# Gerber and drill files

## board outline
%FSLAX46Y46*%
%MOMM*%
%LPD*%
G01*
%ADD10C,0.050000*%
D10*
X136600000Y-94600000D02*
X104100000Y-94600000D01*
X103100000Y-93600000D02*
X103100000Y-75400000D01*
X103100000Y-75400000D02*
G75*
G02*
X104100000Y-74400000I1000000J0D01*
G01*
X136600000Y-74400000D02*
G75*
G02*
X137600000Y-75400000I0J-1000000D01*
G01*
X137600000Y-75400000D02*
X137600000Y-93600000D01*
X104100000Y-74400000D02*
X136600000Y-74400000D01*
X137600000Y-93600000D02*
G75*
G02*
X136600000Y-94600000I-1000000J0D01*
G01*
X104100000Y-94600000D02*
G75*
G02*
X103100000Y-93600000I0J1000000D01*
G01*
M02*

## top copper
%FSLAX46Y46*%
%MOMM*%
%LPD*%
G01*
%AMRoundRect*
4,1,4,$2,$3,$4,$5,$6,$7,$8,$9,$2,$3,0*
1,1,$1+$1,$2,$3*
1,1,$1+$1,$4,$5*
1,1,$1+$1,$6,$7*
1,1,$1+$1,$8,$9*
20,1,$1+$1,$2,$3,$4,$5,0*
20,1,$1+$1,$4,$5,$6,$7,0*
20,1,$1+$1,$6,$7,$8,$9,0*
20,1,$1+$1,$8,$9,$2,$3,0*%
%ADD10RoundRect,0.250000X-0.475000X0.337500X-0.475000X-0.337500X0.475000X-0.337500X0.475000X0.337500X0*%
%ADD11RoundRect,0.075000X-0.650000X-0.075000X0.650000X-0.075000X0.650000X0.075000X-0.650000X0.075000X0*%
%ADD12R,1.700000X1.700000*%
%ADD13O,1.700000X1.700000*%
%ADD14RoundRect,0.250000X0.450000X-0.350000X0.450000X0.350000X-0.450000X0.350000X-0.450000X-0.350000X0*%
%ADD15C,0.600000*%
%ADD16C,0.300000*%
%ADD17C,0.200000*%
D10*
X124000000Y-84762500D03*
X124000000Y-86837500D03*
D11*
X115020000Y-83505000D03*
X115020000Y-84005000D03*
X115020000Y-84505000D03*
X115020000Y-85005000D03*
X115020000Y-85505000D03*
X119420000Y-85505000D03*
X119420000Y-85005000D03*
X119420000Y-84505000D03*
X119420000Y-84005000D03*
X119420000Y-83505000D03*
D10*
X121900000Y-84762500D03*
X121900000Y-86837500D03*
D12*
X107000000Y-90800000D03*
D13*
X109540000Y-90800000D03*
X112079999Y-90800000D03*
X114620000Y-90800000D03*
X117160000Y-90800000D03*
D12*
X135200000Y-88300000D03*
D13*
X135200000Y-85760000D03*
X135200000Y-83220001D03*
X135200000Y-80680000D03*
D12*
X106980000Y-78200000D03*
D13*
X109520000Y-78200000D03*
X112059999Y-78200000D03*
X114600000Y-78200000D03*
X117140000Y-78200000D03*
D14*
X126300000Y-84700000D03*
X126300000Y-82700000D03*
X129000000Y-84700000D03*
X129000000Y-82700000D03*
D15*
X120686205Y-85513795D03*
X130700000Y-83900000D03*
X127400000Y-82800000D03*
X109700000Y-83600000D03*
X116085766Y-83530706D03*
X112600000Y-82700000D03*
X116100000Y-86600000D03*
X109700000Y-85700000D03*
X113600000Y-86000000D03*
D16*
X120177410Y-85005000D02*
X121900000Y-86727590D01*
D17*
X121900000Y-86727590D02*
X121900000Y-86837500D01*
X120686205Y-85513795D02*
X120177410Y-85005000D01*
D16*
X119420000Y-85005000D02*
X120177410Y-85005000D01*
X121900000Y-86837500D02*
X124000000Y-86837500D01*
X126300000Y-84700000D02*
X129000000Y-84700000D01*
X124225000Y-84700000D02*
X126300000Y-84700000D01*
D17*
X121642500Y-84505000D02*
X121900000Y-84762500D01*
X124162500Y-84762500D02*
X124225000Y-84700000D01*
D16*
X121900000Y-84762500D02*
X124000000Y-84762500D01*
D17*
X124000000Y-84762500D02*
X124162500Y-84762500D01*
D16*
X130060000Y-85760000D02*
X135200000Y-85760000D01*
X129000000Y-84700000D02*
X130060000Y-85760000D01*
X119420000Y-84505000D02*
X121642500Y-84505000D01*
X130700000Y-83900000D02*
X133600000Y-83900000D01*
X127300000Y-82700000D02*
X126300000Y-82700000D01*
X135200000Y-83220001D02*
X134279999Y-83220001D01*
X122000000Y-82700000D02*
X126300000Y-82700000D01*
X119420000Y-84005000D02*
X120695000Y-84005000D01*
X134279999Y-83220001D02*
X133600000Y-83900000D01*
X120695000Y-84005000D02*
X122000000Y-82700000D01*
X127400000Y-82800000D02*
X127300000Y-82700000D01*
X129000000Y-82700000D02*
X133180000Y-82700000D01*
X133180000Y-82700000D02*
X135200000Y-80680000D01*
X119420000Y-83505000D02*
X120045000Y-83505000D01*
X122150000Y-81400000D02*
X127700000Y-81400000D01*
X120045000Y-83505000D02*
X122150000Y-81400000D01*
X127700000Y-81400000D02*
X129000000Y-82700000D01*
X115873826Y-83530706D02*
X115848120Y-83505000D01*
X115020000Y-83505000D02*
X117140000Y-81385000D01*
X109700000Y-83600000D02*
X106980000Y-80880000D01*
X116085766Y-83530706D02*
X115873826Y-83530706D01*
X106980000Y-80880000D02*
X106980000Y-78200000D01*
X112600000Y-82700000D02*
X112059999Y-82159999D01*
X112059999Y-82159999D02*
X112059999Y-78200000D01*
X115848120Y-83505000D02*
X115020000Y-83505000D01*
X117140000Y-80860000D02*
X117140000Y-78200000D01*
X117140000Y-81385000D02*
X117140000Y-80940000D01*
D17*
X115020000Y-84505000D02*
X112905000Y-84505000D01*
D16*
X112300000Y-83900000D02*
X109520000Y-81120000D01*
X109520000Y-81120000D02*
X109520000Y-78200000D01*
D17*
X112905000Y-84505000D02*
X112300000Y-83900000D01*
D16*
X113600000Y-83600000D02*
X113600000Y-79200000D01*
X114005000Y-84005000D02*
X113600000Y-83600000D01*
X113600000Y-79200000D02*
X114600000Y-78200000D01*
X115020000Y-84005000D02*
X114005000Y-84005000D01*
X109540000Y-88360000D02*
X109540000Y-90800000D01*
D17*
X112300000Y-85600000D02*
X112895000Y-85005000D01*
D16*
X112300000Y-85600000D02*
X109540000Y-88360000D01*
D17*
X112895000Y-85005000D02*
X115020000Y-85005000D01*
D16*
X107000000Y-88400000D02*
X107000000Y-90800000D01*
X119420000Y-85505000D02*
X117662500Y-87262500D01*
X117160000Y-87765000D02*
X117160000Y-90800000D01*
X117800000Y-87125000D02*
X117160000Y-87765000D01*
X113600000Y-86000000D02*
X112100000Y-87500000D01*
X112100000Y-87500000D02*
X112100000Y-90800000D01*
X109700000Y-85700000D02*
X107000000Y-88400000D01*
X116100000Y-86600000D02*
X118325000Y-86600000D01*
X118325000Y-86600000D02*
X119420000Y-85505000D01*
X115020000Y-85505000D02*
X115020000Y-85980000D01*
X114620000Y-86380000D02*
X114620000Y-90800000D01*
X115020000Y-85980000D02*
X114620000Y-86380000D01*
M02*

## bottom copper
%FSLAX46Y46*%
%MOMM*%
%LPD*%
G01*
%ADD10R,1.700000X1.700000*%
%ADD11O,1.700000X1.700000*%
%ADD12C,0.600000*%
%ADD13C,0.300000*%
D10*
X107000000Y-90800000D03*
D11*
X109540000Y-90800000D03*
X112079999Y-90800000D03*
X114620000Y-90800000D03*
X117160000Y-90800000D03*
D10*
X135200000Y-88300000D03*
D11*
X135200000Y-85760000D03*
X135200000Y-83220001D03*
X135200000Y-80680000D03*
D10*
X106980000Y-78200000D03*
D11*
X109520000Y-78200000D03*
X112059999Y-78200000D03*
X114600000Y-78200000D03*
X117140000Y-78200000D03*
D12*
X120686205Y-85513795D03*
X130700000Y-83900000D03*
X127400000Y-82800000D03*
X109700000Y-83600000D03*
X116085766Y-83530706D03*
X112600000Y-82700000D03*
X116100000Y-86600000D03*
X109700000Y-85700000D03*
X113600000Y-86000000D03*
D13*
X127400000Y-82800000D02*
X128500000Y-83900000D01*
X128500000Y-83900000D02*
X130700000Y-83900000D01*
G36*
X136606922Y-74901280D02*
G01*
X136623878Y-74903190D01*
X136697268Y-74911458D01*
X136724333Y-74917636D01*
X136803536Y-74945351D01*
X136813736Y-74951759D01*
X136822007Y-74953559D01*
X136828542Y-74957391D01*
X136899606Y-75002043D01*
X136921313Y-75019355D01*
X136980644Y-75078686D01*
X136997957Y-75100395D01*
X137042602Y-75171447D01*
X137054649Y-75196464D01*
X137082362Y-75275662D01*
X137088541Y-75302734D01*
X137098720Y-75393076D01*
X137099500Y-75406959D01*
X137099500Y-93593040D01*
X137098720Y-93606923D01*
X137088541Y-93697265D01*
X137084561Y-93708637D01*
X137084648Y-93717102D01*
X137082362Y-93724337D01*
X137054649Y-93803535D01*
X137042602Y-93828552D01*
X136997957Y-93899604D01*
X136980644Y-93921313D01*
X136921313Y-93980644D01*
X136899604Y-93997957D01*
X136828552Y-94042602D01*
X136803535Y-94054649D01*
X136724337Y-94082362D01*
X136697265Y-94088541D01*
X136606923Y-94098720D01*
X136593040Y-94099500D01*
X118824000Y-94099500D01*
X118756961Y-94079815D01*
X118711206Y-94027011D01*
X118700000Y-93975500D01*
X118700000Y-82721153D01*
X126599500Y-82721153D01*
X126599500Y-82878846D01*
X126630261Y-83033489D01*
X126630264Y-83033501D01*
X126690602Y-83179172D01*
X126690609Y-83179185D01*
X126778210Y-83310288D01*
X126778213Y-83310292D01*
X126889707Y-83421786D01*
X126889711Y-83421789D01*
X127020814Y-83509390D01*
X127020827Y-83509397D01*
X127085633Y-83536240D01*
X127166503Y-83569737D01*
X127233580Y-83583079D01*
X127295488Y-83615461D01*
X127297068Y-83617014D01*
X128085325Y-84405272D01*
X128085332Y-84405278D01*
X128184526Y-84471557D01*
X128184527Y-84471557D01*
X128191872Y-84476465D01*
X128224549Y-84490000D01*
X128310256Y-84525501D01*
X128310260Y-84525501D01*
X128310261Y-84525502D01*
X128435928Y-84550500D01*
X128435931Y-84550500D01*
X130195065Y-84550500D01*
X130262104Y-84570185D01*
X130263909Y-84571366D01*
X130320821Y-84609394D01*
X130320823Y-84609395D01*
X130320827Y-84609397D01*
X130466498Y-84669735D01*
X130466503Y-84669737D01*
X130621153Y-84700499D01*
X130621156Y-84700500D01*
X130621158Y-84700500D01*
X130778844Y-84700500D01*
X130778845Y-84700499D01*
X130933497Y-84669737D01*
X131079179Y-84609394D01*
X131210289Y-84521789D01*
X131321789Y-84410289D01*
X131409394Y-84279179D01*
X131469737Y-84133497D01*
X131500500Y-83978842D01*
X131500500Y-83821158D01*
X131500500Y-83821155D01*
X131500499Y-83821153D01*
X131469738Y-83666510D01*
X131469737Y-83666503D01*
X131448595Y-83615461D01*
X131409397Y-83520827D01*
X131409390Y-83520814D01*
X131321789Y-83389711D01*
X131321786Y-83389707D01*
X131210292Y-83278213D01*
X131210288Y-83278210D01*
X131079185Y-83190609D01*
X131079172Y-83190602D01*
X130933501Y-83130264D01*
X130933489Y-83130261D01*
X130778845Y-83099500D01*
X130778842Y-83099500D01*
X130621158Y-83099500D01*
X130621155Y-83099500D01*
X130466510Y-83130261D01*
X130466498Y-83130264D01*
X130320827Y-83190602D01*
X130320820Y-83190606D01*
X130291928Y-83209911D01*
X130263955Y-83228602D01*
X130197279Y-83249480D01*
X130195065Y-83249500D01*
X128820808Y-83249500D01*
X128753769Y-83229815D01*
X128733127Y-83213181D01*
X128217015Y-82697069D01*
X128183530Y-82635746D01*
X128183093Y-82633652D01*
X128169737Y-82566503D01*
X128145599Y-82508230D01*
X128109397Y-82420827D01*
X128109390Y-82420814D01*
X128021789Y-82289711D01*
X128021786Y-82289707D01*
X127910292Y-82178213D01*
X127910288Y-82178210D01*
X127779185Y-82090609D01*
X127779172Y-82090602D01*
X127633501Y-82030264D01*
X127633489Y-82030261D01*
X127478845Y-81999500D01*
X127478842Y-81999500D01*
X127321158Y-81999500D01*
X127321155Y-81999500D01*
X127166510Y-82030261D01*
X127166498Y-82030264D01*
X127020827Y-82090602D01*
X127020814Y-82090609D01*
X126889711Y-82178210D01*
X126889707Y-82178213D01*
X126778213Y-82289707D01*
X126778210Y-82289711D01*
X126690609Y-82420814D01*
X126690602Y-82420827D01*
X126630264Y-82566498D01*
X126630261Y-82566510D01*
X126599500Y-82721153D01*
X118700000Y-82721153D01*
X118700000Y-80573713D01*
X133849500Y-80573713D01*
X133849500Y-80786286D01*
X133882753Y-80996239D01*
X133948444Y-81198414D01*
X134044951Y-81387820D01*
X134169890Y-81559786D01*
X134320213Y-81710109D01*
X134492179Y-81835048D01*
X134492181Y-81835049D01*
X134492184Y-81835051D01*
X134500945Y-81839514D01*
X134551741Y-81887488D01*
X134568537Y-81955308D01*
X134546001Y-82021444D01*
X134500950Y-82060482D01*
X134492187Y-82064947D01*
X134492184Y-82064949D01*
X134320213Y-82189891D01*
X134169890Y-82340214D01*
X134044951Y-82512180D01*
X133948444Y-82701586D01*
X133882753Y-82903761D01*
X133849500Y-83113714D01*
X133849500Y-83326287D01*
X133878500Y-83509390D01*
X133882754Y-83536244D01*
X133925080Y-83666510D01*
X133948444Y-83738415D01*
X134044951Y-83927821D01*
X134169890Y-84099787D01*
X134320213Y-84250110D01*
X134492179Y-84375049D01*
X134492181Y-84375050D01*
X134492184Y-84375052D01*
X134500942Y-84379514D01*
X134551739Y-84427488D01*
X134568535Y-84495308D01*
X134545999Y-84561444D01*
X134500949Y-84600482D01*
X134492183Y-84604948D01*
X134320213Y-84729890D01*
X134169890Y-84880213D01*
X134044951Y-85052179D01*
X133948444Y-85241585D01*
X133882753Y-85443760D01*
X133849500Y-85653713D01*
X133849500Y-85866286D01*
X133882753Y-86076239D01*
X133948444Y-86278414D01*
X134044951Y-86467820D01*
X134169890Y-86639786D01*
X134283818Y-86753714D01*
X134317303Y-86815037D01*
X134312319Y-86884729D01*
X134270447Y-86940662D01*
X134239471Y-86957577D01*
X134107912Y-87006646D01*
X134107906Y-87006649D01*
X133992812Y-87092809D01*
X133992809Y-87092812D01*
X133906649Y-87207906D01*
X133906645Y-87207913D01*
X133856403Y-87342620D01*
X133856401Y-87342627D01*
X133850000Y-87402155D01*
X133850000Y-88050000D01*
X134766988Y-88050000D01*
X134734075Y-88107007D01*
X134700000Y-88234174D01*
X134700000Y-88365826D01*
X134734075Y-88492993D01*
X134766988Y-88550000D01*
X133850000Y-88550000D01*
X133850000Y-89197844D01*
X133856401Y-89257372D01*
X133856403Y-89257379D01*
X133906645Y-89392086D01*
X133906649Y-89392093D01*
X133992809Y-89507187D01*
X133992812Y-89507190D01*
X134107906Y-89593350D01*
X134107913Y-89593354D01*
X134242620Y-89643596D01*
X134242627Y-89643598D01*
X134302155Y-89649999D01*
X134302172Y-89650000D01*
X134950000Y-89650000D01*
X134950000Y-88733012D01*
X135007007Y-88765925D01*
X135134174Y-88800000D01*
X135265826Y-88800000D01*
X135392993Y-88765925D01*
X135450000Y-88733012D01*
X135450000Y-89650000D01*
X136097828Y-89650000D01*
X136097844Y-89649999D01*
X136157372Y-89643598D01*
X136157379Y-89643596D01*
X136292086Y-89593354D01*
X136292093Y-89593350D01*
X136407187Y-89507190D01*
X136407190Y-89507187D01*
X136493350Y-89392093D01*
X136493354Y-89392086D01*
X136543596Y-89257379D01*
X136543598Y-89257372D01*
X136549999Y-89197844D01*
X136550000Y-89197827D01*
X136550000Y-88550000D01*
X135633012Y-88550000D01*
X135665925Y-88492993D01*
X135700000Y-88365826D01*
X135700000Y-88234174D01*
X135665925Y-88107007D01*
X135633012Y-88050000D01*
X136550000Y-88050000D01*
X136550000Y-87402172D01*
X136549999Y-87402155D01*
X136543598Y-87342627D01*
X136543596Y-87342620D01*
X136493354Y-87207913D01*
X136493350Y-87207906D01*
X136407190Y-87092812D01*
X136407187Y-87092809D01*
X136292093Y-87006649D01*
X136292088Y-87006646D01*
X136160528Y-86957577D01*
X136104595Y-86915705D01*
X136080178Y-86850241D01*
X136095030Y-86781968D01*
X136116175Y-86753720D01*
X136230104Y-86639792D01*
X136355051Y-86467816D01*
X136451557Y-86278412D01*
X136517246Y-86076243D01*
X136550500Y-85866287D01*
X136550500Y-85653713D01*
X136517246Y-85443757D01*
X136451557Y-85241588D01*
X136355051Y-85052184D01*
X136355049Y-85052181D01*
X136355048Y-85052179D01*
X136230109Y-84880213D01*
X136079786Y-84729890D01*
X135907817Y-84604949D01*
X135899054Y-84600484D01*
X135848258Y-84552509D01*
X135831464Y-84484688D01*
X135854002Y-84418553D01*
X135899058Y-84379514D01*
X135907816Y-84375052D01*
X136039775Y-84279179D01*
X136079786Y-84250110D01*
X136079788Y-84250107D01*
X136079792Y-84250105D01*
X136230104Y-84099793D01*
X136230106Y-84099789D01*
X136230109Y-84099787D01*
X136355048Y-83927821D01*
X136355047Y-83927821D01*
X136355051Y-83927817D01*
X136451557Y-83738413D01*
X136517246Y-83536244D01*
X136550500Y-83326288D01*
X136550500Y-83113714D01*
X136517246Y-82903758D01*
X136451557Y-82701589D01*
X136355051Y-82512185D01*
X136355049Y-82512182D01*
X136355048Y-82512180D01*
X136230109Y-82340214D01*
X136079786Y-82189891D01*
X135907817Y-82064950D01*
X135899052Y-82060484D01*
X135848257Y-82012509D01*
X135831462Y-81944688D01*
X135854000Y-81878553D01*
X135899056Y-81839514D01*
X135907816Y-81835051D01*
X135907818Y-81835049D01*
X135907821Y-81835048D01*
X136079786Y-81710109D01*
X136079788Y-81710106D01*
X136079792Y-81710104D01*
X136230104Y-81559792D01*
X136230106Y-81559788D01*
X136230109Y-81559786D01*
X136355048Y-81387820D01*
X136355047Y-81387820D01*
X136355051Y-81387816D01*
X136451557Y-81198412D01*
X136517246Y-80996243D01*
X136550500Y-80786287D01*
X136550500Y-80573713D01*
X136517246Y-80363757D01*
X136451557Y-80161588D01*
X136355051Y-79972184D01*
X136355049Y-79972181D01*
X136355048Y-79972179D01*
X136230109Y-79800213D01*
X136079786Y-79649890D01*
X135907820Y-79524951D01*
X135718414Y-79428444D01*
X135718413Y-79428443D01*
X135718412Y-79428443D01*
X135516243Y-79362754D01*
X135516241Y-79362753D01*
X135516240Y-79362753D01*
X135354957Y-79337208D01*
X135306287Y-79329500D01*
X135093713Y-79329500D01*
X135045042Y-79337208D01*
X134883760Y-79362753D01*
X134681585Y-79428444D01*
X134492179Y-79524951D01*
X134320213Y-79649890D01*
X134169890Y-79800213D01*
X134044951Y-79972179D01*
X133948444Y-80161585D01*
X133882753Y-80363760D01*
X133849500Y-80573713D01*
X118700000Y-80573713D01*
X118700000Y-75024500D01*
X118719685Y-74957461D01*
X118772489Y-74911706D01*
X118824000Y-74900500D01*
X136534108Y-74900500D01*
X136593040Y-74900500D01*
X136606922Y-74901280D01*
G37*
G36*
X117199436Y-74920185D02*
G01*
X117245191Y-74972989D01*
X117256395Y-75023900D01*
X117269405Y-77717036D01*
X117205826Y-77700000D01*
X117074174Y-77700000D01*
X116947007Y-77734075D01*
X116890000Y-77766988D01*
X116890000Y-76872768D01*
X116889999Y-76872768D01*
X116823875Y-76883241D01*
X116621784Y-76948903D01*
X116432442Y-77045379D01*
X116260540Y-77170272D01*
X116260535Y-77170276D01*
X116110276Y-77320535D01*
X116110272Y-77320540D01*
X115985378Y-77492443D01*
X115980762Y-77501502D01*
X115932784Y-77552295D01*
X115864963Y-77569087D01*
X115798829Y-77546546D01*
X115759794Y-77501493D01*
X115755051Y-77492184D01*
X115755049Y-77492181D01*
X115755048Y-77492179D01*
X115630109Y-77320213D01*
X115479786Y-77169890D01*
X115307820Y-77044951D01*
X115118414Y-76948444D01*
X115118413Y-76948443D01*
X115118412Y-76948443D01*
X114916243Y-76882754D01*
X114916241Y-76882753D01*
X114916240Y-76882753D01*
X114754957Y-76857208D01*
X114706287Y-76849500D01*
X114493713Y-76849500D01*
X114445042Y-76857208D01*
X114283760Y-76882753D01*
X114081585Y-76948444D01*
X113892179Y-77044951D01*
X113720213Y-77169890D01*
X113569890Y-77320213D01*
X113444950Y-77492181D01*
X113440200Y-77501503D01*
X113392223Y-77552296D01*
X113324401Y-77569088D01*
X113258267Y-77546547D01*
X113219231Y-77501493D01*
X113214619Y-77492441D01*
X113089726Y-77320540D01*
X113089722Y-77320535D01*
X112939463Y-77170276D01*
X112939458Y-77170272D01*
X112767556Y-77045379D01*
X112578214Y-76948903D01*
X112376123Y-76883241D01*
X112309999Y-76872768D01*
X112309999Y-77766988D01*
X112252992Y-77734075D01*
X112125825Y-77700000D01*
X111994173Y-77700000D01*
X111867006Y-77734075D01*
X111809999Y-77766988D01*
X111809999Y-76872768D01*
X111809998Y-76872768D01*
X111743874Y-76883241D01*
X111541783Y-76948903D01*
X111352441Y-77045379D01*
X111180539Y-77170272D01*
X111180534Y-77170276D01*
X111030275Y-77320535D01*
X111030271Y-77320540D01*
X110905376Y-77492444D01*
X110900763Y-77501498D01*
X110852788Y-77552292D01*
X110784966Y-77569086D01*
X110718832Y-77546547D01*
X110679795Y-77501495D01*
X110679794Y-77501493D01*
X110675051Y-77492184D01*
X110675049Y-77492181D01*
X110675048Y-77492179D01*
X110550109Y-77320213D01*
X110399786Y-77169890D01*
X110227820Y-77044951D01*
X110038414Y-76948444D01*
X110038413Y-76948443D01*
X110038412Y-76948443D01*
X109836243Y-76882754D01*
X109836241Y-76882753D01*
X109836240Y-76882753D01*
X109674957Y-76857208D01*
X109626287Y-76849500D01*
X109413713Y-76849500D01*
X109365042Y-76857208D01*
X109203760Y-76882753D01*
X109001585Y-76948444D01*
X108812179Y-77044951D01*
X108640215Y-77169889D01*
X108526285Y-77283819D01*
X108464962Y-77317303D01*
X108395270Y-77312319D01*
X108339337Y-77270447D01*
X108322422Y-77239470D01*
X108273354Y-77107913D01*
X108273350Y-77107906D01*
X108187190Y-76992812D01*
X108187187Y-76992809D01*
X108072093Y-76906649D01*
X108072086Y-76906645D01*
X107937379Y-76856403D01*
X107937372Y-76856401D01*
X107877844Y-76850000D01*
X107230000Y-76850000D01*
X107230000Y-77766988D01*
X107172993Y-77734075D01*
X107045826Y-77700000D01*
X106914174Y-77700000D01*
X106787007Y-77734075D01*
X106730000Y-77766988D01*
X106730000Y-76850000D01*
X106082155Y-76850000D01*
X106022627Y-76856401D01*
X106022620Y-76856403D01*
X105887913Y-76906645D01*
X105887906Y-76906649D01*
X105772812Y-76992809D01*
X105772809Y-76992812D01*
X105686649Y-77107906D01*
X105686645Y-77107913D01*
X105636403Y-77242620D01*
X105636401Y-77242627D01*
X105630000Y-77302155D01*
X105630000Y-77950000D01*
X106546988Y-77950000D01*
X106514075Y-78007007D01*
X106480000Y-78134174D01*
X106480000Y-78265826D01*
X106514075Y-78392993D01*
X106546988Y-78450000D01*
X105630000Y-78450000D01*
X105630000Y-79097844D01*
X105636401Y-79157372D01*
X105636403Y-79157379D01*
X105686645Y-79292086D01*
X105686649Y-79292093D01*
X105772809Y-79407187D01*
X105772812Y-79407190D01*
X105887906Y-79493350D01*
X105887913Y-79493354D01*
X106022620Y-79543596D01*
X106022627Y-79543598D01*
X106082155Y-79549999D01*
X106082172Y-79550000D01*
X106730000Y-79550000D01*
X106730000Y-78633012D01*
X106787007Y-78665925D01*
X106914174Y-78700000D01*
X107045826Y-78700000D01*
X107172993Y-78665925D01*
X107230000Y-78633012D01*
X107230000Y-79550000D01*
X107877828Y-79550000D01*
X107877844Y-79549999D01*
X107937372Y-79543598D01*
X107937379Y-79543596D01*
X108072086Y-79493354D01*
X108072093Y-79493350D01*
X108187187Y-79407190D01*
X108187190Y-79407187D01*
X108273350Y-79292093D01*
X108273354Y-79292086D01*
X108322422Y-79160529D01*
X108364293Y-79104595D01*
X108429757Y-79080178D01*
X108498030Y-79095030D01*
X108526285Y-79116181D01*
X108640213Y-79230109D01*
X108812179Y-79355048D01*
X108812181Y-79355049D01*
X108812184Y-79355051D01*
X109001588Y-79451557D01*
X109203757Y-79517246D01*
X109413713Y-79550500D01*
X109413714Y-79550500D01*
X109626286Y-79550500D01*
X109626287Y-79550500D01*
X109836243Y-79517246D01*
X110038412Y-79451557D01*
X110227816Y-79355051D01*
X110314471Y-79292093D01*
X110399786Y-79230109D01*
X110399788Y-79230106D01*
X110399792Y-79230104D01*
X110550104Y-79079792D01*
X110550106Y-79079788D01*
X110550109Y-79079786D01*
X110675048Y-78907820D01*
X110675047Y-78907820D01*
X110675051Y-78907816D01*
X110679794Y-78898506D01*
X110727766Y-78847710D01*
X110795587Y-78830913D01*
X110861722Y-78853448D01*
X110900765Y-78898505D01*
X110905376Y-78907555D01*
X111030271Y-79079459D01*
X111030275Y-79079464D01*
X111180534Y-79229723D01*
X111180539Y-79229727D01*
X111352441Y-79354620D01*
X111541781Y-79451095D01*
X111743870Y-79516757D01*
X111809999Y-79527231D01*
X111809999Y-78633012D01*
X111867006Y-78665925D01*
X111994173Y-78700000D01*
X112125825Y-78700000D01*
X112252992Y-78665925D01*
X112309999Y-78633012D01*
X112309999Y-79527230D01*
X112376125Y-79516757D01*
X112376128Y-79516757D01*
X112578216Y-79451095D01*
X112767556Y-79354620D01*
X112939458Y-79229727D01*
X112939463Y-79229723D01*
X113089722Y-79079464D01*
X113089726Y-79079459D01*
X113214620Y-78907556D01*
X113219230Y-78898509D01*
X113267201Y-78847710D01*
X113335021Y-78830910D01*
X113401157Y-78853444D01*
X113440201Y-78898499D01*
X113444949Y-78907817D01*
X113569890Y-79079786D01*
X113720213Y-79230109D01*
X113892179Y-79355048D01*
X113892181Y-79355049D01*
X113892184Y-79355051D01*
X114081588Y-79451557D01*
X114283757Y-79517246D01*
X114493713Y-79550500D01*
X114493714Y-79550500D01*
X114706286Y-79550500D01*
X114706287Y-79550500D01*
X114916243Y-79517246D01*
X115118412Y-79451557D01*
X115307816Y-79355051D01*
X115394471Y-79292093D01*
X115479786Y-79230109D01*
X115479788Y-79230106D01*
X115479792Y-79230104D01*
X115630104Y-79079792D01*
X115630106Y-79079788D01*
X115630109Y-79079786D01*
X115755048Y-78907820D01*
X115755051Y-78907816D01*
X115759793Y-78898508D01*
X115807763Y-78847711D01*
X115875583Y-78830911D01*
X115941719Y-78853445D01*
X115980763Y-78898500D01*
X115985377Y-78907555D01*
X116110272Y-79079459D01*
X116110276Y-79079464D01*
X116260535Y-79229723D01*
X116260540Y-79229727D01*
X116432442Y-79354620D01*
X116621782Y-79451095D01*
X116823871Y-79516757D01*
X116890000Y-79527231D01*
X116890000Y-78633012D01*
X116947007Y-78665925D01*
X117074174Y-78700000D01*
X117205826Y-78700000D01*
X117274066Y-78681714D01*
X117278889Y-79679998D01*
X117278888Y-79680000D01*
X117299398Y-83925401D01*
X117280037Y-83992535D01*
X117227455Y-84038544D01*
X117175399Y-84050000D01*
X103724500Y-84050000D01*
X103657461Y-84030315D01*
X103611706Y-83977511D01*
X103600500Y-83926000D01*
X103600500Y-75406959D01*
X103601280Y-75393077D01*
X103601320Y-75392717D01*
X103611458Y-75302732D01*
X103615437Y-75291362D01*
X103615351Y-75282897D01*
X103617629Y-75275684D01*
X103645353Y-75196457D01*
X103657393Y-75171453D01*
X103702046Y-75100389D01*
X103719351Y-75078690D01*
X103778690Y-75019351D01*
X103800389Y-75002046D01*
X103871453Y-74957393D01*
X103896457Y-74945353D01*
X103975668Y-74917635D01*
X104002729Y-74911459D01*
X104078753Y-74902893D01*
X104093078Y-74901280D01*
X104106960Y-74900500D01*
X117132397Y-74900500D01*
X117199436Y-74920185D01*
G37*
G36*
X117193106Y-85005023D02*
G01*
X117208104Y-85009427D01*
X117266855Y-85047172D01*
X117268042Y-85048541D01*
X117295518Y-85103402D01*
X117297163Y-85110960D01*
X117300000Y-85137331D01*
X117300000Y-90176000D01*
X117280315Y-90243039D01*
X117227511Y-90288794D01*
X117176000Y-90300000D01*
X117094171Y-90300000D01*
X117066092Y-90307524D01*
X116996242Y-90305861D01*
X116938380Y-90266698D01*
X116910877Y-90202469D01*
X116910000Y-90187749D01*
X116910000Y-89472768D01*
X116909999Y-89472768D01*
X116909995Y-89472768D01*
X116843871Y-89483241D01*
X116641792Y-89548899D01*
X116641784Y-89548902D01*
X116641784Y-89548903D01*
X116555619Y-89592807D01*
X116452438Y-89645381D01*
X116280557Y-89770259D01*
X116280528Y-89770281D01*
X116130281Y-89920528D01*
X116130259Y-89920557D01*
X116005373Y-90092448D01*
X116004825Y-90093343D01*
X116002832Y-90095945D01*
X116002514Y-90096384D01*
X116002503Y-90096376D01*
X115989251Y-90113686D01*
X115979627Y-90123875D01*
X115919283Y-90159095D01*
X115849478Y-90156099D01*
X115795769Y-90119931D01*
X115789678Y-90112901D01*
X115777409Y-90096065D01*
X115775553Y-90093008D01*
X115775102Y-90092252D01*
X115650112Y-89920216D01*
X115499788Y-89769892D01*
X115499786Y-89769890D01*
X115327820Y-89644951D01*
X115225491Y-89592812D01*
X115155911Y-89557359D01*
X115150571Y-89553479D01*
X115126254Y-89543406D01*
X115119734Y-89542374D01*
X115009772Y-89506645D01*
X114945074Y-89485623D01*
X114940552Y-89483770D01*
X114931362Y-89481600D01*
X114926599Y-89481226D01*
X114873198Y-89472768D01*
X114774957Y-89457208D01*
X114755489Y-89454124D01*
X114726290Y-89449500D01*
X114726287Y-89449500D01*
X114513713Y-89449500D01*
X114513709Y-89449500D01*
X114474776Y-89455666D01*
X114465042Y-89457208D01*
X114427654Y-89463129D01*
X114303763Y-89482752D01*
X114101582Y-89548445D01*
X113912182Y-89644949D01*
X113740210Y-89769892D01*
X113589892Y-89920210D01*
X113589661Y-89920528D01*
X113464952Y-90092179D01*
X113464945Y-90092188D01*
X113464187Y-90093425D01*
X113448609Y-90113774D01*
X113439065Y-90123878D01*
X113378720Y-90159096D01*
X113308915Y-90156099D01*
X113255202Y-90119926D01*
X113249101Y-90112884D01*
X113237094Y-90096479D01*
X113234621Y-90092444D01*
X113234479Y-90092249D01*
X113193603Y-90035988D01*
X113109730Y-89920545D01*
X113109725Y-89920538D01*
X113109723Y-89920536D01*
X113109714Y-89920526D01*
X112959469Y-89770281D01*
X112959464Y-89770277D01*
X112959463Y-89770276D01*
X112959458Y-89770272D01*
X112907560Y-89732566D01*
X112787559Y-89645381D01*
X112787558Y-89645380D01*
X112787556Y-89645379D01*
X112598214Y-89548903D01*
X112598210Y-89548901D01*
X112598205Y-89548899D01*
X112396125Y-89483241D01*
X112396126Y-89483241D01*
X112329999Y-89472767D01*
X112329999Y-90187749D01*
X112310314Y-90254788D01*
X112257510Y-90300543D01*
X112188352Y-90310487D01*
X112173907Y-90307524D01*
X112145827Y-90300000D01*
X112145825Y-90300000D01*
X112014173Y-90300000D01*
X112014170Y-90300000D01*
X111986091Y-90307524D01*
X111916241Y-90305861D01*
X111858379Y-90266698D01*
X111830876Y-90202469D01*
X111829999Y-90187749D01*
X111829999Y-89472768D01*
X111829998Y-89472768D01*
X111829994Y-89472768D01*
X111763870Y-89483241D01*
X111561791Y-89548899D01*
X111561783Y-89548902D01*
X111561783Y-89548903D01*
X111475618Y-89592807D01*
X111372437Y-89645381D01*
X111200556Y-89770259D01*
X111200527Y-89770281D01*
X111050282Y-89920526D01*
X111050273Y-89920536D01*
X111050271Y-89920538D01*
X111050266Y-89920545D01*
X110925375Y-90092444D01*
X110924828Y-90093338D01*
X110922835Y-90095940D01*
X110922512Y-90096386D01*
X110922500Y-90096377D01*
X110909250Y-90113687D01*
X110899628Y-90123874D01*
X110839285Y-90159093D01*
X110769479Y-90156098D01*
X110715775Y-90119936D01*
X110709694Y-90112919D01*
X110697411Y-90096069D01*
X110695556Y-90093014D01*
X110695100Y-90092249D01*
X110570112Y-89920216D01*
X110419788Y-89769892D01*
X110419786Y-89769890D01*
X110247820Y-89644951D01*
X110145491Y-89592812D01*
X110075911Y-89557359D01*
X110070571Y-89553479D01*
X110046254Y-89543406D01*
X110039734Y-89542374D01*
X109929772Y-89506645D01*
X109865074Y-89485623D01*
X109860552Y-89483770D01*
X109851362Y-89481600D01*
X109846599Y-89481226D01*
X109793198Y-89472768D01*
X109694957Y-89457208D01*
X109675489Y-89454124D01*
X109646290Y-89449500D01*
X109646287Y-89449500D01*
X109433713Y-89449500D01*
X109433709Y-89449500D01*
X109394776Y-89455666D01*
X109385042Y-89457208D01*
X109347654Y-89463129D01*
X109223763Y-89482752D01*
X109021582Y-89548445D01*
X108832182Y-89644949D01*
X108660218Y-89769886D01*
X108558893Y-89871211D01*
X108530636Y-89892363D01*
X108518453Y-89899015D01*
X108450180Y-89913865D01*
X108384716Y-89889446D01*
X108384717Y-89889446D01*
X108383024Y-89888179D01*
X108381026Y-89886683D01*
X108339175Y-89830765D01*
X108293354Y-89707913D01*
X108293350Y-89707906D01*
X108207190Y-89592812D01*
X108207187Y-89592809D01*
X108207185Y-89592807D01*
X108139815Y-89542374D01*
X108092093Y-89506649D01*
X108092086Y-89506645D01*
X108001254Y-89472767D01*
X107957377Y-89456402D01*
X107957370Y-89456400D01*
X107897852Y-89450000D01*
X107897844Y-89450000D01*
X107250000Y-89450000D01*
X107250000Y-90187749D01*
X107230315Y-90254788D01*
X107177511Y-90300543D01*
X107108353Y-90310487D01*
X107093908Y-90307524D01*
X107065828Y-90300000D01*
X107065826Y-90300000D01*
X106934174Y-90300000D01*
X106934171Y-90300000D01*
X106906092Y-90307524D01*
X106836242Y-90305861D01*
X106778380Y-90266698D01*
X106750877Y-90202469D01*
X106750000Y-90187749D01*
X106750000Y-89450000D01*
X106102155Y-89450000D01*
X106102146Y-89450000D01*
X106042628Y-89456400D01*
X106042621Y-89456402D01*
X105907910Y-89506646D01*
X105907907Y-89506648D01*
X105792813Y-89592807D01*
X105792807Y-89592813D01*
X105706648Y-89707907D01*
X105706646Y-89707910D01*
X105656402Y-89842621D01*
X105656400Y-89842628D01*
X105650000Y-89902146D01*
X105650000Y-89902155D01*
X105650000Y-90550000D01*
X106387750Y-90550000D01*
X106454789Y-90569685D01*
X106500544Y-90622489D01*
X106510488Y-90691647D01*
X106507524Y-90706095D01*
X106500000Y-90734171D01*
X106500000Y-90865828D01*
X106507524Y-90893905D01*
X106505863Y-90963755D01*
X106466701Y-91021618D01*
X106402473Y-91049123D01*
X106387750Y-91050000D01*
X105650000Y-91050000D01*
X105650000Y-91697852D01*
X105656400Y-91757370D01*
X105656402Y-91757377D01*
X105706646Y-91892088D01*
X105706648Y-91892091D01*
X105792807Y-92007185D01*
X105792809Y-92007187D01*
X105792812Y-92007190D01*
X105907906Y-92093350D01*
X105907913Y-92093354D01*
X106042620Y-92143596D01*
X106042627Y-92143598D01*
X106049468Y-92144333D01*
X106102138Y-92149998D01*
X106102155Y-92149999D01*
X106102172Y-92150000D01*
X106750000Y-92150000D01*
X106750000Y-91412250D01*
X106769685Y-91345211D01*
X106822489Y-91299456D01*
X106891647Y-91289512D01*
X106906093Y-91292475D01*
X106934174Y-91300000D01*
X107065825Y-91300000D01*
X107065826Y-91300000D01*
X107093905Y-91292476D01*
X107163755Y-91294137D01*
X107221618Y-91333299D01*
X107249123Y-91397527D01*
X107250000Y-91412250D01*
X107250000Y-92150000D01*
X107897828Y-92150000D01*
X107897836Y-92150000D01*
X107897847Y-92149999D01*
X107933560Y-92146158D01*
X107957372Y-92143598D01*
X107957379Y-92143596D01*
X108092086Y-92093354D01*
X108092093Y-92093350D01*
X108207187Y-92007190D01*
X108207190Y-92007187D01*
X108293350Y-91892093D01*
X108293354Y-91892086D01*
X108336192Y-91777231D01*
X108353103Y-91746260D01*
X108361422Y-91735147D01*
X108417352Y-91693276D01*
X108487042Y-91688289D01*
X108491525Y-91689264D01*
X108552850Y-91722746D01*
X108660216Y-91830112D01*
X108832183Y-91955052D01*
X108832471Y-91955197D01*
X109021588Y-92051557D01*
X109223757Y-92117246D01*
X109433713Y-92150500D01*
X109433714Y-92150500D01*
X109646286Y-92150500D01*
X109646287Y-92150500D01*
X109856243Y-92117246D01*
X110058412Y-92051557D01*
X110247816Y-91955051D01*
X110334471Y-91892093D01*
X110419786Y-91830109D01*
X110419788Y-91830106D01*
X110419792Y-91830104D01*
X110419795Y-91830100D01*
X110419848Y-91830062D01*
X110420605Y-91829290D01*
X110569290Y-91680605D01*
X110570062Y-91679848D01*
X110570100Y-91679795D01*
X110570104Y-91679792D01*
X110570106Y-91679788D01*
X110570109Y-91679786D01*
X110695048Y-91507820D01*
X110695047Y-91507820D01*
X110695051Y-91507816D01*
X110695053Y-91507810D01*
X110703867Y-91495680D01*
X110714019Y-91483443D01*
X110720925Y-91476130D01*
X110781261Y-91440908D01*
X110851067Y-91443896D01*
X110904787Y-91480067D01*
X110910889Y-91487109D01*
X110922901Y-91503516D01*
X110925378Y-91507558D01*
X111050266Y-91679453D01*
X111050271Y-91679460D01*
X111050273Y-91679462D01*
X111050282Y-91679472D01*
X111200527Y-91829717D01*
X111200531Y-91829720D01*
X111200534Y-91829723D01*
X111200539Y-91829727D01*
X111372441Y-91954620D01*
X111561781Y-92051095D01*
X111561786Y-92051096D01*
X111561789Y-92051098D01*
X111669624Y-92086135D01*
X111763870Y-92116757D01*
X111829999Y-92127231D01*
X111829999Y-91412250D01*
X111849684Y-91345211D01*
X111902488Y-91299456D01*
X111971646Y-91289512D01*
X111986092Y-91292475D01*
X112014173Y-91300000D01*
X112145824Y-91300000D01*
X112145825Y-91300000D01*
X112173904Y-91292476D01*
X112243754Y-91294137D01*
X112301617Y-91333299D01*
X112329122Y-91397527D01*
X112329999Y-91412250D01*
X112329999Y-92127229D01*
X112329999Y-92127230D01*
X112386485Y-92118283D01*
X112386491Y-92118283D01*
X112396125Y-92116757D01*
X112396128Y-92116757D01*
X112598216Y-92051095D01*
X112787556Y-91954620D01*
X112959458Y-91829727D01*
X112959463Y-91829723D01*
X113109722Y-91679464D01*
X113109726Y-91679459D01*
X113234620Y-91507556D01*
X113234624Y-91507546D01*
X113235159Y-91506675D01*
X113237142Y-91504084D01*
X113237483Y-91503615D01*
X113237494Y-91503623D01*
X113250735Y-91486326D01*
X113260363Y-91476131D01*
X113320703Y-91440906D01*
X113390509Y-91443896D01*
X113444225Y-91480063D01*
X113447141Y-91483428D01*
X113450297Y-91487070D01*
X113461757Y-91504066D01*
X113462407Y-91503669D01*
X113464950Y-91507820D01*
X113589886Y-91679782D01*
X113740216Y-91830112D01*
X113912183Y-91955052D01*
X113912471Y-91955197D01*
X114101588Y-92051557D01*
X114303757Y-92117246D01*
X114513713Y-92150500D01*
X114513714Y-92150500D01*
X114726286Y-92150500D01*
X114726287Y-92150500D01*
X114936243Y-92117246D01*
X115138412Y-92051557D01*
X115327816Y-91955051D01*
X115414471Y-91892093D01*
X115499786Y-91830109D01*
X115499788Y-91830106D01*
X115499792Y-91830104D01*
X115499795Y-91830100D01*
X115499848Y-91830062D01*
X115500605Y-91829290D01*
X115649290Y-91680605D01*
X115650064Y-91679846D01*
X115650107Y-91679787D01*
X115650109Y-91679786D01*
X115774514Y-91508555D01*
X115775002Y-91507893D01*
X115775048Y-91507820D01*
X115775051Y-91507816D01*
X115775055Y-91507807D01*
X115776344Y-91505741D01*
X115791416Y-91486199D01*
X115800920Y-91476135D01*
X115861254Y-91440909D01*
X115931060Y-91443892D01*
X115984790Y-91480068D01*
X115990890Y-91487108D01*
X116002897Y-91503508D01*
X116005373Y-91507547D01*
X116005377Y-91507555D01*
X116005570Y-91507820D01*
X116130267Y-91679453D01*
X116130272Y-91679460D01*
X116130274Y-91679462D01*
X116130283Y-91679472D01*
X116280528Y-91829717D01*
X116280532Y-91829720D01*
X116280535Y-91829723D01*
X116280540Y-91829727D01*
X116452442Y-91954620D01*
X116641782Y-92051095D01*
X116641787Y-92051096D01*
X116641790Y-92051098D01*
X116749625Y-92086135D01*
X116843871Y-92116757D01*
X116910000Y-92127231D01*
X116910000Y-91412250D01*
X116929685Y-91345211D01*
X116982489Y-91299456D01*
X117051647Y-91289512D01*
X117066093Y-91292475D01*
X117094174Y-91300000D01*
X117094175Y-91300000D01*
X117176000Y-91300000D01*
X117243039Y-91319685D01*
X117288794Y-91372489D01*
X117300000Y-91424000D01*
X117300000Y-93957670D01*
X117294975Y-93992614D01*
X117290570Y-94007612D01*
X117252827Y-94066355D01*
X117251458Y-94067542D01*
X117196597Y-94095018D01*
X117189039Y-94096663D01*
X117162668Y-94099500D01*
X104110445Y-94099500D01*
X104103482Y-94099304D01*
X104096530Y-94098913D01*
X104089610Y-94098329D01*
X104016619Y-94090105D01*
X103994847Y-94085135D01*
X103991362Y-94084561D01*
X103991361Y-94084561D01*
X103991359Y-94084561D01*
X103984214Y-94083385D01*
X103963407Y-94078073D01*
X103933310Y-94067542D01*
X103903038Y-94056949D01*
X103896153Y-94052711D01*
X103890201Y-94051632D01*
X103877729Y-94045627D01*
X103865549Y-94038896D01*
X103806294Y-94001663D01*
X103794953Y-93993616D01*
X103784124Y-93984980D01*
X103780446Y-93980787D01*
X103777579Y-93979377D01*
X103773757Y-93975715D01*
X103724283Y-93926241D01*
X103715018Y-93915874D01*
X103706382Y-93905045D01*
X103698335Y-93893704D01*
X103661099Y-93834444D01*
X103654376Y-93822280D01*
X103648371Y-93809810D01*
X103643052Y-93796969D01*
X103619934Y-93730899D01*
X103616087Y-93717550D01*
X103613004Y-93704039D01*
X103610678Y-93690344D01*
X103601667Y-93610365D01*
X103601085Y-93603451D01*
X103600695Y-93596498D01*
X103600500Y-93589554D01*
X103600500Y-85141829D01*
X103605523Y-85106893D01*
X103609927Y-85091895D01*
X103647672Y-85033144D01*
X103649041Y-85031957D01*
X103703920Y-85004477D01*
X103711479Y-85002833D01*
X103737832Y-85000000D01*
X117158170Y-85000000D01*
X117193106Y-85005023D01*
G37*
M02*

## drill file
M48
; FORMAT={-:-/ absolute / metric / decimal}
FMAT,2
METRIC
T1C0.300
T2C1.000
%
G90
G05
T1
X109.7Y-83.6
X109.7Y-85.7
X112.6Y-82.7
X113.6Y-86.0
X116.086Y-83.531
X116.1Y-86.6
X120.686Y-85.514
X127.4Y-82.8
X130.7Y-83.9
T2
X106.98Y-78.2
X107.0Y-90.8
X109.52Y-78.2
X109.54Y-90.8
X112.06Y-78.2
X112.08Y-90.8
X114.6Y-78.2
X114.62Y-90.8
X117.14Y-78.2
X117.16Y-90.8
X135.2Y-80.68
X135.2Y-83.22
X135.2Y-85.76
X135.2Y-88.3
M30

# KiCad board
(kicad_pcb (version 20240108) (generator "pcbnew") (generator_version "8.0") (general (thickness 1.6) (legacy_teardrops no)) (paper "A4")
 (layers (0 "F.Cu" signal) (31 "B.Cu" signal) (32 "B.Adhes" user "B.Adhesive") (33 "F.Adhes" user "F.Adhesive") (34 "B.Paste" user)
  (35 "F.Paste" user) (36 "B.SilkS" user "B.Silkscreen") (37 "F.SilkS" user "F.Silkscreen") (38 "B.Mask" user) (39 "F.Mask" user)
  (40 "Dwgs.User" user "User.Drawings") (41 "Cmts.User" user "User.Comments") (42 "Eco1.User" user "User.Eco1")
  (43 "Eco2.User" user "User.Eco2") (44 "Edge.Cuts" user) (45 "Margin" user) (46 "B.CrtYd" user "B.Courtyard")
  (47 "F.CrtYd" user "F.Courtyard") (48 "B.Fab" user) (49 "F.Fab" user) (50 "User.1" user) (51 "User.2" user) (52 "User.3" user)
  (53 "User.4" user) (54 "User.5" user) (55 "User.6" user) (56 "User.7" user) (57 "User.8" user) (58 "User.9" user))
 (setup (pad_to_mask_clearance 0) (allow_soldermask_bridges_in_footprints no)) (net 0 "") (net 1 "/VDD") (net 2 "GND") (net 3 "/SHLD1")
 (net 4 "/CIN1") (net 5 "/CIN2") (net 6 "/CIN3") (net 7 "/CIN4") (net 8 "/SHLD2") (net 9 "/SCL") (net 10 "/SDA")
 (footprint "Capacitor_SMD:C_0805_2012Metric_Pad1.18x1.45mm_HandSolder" (layer "F.Cu") (at 124 85.8 -90)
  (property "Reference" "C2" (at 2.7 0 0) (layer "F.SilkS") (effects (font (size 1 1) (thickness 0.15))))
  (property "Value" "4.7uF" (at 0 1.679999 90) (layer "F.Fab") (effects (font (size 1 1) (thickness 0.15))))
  (pad "1" smd roundrect (at -1.0375 0 270) (size 1.175 1.45) (layers "F.Cu" "F.Paste" "F.Mask") (roundrect_rratio 0.212766) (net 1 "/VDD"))
  (pad "2" smd roundrect (at 1.0375 0 270) (size 1.175 1.45) (layers "F.Cu" "F.Paste" "F.Mask") (roundrect_rratio 0.212766) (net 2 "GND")))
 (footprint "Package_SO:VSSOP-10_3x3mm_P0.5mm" (layer "F.Cu") (at 117.22 84.505)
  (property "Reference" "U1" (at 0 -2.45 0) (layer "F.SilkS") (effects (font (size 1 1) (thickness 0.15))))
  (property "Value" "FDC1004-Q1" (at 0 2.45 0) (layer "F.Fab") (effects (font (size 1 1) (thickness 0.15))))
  (pad "1" smd roundrect (at -2.2 -1) (size 1.45 0.3) (layers "F.Cu" "F.Paste" "F.Mask") (roundrect_rratio 0.25) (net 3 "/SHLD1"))
  (pad "2" smd roundrect (at -2.2 -0.5) (size 1.45 0.3) (layers "F.Cu" "F.Paste" "F.Mask") (roundrect_rratio 0.25) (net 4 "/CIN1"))
  (pad "3" smd roundrect (at -2.2 0) (size 1.45 0.3) (layers "F.Cu" "F.Paste" "F.Mask") (roundrect_rratio 0.25) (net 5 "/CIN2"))
  (pad "4" smd roundrect (at -2.2 0.5) (size 1.45 0.3) (layers "F.Cu" "F.Paste" "F.Mask") (roundrect_rratio 0.25) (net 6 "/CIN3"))
  (pad "5" smd roundrect (at -2.2 1) (size 1.45 0.3) (layers "F.Cu" "F.Paste" "F.Mask") (roundrect_rratio 0.25) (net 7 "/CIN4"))
  (pad "6" smd roundrect (at 2.2 1) (size 1.45 0.3) (layers "F.Cu" "F.Paste" "F.Mask") (roundrect_rratio 0.25) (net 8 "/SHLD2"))
  (pad "7" smd roundrect (at 2.2 0.5) (size 1.45 0.3) (layers "F.Cu" "F.Paste" "F.Mask") (roundrect_rratio 0.25) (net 2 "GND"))
  (pad "8" smd roundrect (at 2.2 0) (size 1.45 0.3) (layers "F.Cu" "F.Paste" "F.Mask") (roundrect_rratio 0.25) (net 1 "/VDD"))
  (pad "9" smd roundrect (at 2.2 -0.5) (size 1.45 0.3) (layers "F.Cu" "F.Paste" "F.Mask") (roundrect_rratio 0.25) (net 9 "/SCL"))
  (pad "10" smd roundrect (at 2.2 -1) (size 1.45 0.3) (layers "F.Cu" "F.Paste" "F.Mask") (roundrect_rratio 0.25) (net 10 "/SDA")))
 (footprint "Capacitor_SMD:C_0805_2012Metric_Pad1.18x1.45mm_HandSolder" (layer "F.Cu") (at 121.9 85.8 -90)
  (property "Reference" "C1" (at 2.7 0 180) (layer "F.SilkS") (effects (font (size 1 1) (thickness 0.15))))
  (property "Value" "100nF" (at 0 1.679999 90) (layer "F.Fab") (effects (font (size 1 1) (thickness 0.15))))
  (pad "1" smd roundrect (at -1.0375 0 270) (size 1.175 1.45) (layers "F.Cu" "F.Paste" "F.Mask") (roundrect_rratio 0.212766) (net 1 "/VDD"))
  (pad "2" smd roundrect (at 1.0375 0 270) (size 1.175 1.45) (layers "F.Cu" "F.Paste" "F.Mask") (roundrect_rratio 0.212766) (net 2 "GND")))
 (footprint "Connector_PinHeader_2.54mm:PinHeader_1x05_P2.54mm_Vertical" (layer "F.Cu") (at 107 90.8 90)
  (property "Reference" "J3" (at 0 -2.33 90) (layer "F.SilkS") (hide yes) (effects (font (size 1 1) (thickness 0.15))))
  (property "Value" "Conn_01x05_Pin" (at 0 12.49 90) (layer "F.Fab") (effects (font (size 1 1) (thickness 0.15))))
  (pad "1" thru_hole rect (at 0 0 90) (size 1.7 1.7) (drill 1) (layers "*.Cu" "*.Mask") (remove_unused_layers no) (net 8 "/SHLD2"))
  (pad "2" thru_hole oval (at 0 2.54 90) (size 1.7 1.7) (drill 1) (layers "*.Cu" "*.Mask") (remove_unused_layers no) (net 6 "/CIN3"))
  (pad "3" thru_hole oval (at 0 5.079999 90) (size 1.7 1.7) (drill 1) (layers "*.Cu" "*.Mask") (remove_unused_layers no) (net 8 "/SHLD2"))
  (pad "4" thru_hole oval (at 0 7.62 90) (size 1.7 1.7) (drill 1) (layers "*.Cu" "*.Mask") (remove_unused_layers no) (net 7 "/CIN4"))
  (pad "5" thru_hole oval (at 0 10.16 90) (size 1.7 1.7) (drill 1) (layers "*.Cu" "*.Mask") (remove_unused_layers no) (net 8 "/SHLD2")))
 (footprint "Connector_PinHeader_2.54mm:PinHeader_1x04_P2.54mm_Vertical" (layer "F.Cu") (at 135.2 88.3 180)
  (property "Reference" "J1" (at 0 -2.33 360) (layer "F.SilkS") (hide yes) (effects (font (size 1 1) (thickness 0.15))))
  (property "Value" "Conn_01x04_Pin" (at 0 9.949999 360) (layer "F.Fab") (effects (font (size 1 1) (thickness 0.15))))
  (pad "1" thru_hole rect (at 0 0 180) (size 1.7 1.7) (drill 1) (layers "*.Cu" "*.Mask") (remove_unused_layers no) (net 2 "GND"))
  (pad "2" thru_hole oval (at 0 2.54 180) (size 1.7 1.7) (drill 1) (layers "*.Cu" "*.Mask") (remove_unused_layers no) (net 1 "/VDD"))
  (pad "3" thru_hole oval (at 0 5.079999 180) (size 1.7 1.7) (drill 1) (layers "*.Cu" "*.Mask") (remove_unused_layers no) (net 9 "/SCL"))
  (pad "4" thru_hole oval (at 0 7.62 180) (size 1.7 1.7) (drill 1) (layers "*.Cu" "*.Mask") (remove_unused_layers no) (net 10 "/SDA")))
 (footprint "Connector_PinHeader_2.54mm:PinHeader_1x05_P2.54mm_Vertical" (layer "F.Cu") (at 106.98 78.2 90)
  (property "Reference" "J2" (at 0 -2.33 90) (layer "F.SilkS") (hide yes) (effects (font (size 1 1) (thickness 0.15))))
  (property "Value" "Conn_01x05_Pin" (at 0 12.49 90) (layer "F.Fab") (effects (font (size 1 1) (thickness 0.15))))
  (pad "1" thru_hole rect (at 0 0 90) (size 1.7 1.7) (drill 1) (layers "*.Cu" "*.Mask") (remove_unused_layers no) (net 3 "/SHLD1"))
  (pad "2" thru_hole oval (at 0 2.54 90) (size 1.7 1.7) (drill 1) (layers "*.Cu" "*.Mask") (remove_unused_layers no) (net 5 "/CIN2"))
  (pad "3" thru_hole oval (at 0 5.079999 90) (size 1.7 1.7) (drill 1) (layers "*.Cu" "*.Mask") (remove_unused_layers no) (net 3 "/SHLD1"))
  (pad "4" thru_hole oval (at 0 7.62 90) (size 1.7 1.7) (drill 1) (layers "*.Cu" "*.Mask") (remove_unused_layers no) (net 4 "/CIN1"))
  (pad "5" thru_hole oval (at 0 10.16 90) (size 1.7 1.7) (drill 1) (layers "*.Cu" "*.Mask") (remove_unused_layers no) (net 3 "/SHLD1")))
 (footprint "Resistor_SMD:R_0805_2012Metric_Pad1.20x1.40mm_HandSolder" (layer "F.Cu") (at 126.3 83.7 90)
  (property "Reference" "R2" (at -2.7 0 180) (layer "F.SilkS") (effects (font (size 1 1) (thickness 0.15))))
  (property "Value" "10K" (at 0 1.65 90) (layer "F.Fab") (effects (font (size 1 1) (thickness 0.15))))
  (pad "1" smd roundrect (at -1 0 90) (size 1.2 1.4) (layers "F.Cu" "F.Paste" "F.Mask") (roundrect_rratio 0.208333) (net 1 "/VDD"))
  (pad "2" smd roundrect (at 1 0 90) (size 1.2 1.4) (layers "F.Cu" "F.Paste" "F.Mask") (roundrect_rratio 0.208333) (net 9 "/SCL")))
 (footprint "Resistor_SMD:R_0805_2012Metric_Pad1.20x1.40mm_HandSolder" (layer "F.Cu") (at 129 83.7 90)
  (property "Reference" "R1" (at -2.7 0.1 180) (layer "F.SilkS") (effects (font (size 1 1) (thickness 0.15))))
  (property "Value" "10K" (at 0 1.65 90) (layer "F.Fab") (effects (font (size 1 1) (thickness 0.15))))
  (pad "1" smd roundrect (at -1 0 90) (size 1.2 1.4) (layers "F.Cu" "F.Paste" "F.Mask") (roundrect_rratio 0.208333) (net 1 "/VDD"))
  (pad "2" smd roundrect (at 1 0 90) (size 1.2 1.4) (layers "F.Cu" "F.Paste" "F.Mask") (roundrect_rratio 0.208333) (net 10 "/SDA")))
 (gr_line (start 136.6 94.6) (end 104.1 94.6) (stroke (width 0.05) (type default)) (layer "Edge.Cuts"))
 (gr_line (start 103.1 93.6) (end 103.1 75.4) (stroke (width 0.05) (type default)) (layer "Edge.Cuts"))
 (gr_arc (start 103.1 75.4) (mid 103.392893 74.692893) (end 104.1 74.4) (stroke (width 0.05) (type default)) (layer "Edge.Cuts"))
 (gr_arc (start 136.6 74.4) (mid 137.307107 74.692893) (end 137.6 75.4) (stroke (width 0.05) (type default)) (layer "Edge.Cuts"))
 (gr_line (start 137.6 75.4) (end 137.6 93.6) (stroke (width 0.05) (type default)) (layer "Edge.Cuts"))
 (gr_line (start 104.1 74.4) (end 136.6 74.4) (stroke (width 0.05) (type default)) (layer "Edge.Cuts"))
 (gr_arc (start 137.6 93.6) (mid 137.307107 94.307107) (end 136.6 94.6) (stroke (width 0.05) (type default)) (layer "Edge.Cuts"))
 (gr_arc (start 104.1 94.6) (mid 103.392893 94.307107) (end 103.1 93.6) (stroke (width 0.05) (type default)) (layer "Edge.Cuts"))
 (segment (start 120.17741 85.005) (end 121.9 86.72759) (width 0.3) (layer "F.Cu") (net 2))
 (segment (start 121.9 86.72759) (end 121.9 86.8375) (width 0.2) (layer "F.Cu") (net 2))
 (segment (start 120.686205 85.513795) (end 120.17741 85.005) (width 0.2) (layer "F.Cu") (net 2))
 (segment (start 119.42 85.005) (end 120.17741 85.005) (width 0.3) (layer "F.Cu") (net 2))
 (segment (start 121.9 86.8375) (end 124 86.8375) (width 0.3) (layer "F.Cu") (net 2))
 (via (at 120.686205 85.513795) (size 0.6) (drill 0.3) (layers "F.Cu" "B.Cu") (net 2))
 (segment (start 126.3 84.7) (end 129 84.7) (width 0.3) (layer "F.Cu") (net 1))
 (segment (start 124.225 84.7) (end 126.3 84.7) (width 0.3) (layer "F.Cu") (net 1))
 (segment (start 121.6425 84.505) (end 121.9 84.7625) (width 0.2) (layer "F.Cu") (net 1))
 (segment (start 124.1625 84.7625) (end 124.225 84.7) (width 0.2) (layer "F.Cu") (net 1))
 (segment (start 121.9 84.7625) (end 124 84.7625) (width 0.3) (layer "F.Cu") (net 1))
 (segment (start 124 84.7625) (end 124.1625 84.7625) (width 0.2) (layer "F.Cu") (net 1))
 (segment (start 130.06 85.76) (end 135.2 85.76) (width 0.3) (layer "F.Cu") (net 1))
 (segment (start 129 84.7) (end 130.06 85.76) (width 0.3) (layer "F.Cu") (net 1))
 (segment (start 119.42 84.505) (end 121.6425 84.505) (width 0.3) (layer "F.Cu") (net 1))
 (segment (start 130.7 83.9) (end 133.6 83.9) (width 0.3) (layer "F.Cu") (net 9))
 (segment (start 127.3 82.7) (end 126.3 82.7) (width 0.3) (layer "F.Cu") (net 9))
 (segment (start 135.2 83.220001) (end 134.279999 83.220001) (width 0.3) (layer "F.Cu") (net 9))
 (segment (start 122 82.7) (end 126.3 82.7) (width 0.3) (layer "F.Cu") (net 9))
 (segment (start 119.42 84.005) (end 120.695 84.005) (width 0.3) (layer "F.Cu") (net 9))
 (segment (start 134.279999 83.220001) (end 133.6 83.9) (width 0.3) (layer "F.Cu") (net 9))
 (segment (start 120.695 84.005) (end 122 82.7) (width 0.3) (layer "F.Cu") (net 9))
 (segment (start 127.4 82.8) (end 127.3 82.7) (width 0.3) (layer "F.Cu") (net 9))
 (via (at 130.7 83.9) (size 0.6) (drill 0.3) (layers "F.Cu" "B.Cu") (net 9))
 (via (at 127.4 82.8) (size 0.6) (drill 0.3) (layers "F.Cu" "B.Cu") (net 9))
 (segment (start 127.4 82.8) (end 128.5 83.9) (width 0.3) (layer "B.Cu") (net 9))
 (segment (start 128.5 83.9) (end 130.7 83.9) (width 0.3) (layer "B.Cu") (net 9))
 (segment (start 129 82.7) (end 133.18 82.7) (width 0.3) (layer "F.Cu") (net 10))
 (segment (start 133.18 82.7) (end 135.2 80.68) (width 0.3) (layer "F.Cu") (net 10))
 (segment (start 119.42 83.505) (end 120.045 83.505) (width 0.3) (layer "F.Cu") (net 10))
 (segment (start 122.15 81.4) (end 127.7 81.4) (width 0.3) (layer "F.Cu") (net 10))
 (segment (start 120.045 83.505) (end 122.15 81.4) (width 0.3) (layer "F.Cu") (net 10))
 (segment (start 127.7 81.4) (end 129 82.7) (width 0.3) (layer "F.Cu") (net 10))
 (segment (start 115.873826 83.530706) (end 115.84812 83.505) (width 0.3) (layer "F.Cu") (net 3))
 (segment (start 115.02 83.505) (end 117.14 81.385) (width 0.3) (layer "F.Cu") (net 3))
 (segment (start 109.7 83.6) (end 106.98 80.88) (width 0.3) (layer "F.Cu") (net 3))
 (segment (start 116.085766 83.530706) (end 115.873826 83.530706) (width 0.3) (layer "F.Cu") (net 3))
 (segment (start 106.98 80.88) (end 106.98 78.2) (width 0.3) (layer "F.Cu") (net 3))
 (segment (start 112.6 82.7) (end 112.059999 82.159999) (width 0.3) (layer "F.Cu") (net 3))
 (segment (start 112.059999 82.159999) (end 112.059999 78.2) (width 0.3) (layer "F.Cu") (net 3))
 (segment (start 115.84812 83.505) (end 115.02 83.505) (width 0.3) (layer "F.Cu") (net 3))
 (segment (start 117.14 80.86) (end 117.14 78.2) (width 0.3) (layer "F.Cu") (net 3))
 (segment (start 117.14 81.385) (end 117.14 80.94) (width 0.3) (layer "F.Cu") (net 3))
 (via (at 109.7 83.6) (size 0.6) (drill 0.3) (layers "F.Cu" "B.Cu") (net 3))
 (via (at 116.085766 83.530706) (size 0.6) (drill 0.3) (layers "F.Cu" "B.Cu") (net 3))
 (via (at 112.6 82.7) (size 0.6) (drill 0.3) (layers "F.Cu" "B.Cu") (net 3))
 (segment (start 115.02 84.505) (end 112.905 84.505) (width 0.2) (layer "F.Cu") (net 5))
 (segment (start 112.3 83.9) (end 109.52 81.12) (width 0.3) (layer "F.Cu") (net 5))
 (segment (start 109.52 81.12) (end 109.52 78.2) (width 0.3) (layer "F.Cu") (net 5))
 (segment (start 112.905 84.505) (end 112.3 83.9) (width 0.2) (layer "F.Cu") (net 5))
 (segment (start 113.6 83.6) (end 113.6 79.2) (width 0.3) (layer "F.Cu") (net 4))
 (segment (start 114.005 84.005) (end 113.6 83.6) (width 0.3) (layer "F.Cu") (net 4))
 (segment (start 113.6 79.2) (end 114.6 78.2) (width 0.3) (layer "F.Cu") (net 4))
 (segment (start 115.02 84.005) (end 114.005 84.005) (width 0.3) (layer "F.Cu") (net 4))
 (segment (start 109.54 88.36) (end 109.54 90.8) (width 0.3) (layer "F.Cu") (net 6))
 (segment (start 112.3 85.6) (end 112.895 85.005) (width 0.2) (layer "F.Cu") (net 6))
 (segment (start 112.3 85.6) (end 109.54 88.36) (width 0.3) (layer "F.Cu") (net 6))
 (segment (start 112.895 85.005) (end 115.02 85.005) (width 0.2) (layer "F.Cu") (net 6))
 (segment (start 107 88.4) (end 107 90.8) (width 0.3) (layer "F.Cu") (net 8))
 (segment (start 119.42 85.505) (end 117.6625 87.2625) (width 0.3) (layer "F.Cu") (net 8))
 (segment (start 117.16 87.765) (end 117.16 90.8) (width 0.3) (layer "F.Cu") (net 8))
 (segment (start 117.8 87.125) (end 117.16 87.765) (width 0.3) (layer "F.Cu") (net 8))
 (segment (start 113.6 86) (end 112.1 87.5) (width 0.3) (layer "F.Cu") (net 8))
 (segment (start 112.1 87.5) (end 112.1 90.8) (width 0.3) (layer "F.Cu") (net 8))
 (segment (start 109.7 85.7) (end 107 88.4) (width 0.3) (layer "F.Cu") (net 8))
 (segment (start 116.1 86.6) (end 118.325 86.6) (width 0.3) (layer "F.Cu") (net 8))
 (segment (start 118.325 86.6) (end 119.42 85.505) (width 0.3) (layer "F.Cu") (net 8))
 (via (at 116.1 86.6) (size 0.6) (drill 0.3) (layers "F.Cu" "B.Cu") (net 8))
 (via (at 109.7 85.7) (size 0.6) (drill 0.3) (layers "F.Cu" "B.Cu") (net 8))
 (via (at 113.6 86) (size 0.6) (drill 0.3) (layers "F.Cu" "B.Cu") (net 8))
 (segment (start 115.02 85.505) (end 115.02 85.98) (width 0.3) (layer "F.Cu") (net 7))
 (segment (start 114.62 86.38) (end 114.62 90.8) (width 0.3) (layer "F.Cu") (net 7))
 (segment (start 115.02 85.98) (end 114.62 86.38) (width 0.3) (layer "F.Cu") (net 7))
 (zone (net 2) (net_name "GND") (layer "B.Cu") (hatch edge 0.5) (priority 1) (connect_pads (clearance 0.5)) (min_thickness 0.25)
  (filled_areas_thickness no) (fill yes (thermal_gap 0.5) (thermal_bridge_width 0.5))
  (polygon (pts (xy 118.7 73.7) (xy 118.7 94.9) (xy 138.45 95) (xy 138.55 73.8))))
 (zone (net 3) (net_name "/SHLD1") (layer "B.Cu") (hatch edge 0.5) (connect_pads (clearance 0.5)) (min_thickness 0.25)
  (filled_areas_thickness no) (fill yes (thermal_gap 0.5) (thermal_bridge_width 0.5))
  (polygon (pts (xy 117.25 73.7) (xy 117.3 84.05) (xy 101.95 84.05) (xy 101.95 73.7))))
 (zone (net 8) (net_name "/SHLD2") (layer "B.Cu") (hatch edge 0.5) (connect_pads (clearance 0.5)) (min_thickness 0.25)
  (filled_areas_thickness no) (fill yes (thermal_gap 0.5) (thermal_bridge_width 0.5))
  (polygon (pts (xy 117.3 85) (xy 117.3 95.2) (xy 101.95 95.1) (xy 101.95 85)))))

